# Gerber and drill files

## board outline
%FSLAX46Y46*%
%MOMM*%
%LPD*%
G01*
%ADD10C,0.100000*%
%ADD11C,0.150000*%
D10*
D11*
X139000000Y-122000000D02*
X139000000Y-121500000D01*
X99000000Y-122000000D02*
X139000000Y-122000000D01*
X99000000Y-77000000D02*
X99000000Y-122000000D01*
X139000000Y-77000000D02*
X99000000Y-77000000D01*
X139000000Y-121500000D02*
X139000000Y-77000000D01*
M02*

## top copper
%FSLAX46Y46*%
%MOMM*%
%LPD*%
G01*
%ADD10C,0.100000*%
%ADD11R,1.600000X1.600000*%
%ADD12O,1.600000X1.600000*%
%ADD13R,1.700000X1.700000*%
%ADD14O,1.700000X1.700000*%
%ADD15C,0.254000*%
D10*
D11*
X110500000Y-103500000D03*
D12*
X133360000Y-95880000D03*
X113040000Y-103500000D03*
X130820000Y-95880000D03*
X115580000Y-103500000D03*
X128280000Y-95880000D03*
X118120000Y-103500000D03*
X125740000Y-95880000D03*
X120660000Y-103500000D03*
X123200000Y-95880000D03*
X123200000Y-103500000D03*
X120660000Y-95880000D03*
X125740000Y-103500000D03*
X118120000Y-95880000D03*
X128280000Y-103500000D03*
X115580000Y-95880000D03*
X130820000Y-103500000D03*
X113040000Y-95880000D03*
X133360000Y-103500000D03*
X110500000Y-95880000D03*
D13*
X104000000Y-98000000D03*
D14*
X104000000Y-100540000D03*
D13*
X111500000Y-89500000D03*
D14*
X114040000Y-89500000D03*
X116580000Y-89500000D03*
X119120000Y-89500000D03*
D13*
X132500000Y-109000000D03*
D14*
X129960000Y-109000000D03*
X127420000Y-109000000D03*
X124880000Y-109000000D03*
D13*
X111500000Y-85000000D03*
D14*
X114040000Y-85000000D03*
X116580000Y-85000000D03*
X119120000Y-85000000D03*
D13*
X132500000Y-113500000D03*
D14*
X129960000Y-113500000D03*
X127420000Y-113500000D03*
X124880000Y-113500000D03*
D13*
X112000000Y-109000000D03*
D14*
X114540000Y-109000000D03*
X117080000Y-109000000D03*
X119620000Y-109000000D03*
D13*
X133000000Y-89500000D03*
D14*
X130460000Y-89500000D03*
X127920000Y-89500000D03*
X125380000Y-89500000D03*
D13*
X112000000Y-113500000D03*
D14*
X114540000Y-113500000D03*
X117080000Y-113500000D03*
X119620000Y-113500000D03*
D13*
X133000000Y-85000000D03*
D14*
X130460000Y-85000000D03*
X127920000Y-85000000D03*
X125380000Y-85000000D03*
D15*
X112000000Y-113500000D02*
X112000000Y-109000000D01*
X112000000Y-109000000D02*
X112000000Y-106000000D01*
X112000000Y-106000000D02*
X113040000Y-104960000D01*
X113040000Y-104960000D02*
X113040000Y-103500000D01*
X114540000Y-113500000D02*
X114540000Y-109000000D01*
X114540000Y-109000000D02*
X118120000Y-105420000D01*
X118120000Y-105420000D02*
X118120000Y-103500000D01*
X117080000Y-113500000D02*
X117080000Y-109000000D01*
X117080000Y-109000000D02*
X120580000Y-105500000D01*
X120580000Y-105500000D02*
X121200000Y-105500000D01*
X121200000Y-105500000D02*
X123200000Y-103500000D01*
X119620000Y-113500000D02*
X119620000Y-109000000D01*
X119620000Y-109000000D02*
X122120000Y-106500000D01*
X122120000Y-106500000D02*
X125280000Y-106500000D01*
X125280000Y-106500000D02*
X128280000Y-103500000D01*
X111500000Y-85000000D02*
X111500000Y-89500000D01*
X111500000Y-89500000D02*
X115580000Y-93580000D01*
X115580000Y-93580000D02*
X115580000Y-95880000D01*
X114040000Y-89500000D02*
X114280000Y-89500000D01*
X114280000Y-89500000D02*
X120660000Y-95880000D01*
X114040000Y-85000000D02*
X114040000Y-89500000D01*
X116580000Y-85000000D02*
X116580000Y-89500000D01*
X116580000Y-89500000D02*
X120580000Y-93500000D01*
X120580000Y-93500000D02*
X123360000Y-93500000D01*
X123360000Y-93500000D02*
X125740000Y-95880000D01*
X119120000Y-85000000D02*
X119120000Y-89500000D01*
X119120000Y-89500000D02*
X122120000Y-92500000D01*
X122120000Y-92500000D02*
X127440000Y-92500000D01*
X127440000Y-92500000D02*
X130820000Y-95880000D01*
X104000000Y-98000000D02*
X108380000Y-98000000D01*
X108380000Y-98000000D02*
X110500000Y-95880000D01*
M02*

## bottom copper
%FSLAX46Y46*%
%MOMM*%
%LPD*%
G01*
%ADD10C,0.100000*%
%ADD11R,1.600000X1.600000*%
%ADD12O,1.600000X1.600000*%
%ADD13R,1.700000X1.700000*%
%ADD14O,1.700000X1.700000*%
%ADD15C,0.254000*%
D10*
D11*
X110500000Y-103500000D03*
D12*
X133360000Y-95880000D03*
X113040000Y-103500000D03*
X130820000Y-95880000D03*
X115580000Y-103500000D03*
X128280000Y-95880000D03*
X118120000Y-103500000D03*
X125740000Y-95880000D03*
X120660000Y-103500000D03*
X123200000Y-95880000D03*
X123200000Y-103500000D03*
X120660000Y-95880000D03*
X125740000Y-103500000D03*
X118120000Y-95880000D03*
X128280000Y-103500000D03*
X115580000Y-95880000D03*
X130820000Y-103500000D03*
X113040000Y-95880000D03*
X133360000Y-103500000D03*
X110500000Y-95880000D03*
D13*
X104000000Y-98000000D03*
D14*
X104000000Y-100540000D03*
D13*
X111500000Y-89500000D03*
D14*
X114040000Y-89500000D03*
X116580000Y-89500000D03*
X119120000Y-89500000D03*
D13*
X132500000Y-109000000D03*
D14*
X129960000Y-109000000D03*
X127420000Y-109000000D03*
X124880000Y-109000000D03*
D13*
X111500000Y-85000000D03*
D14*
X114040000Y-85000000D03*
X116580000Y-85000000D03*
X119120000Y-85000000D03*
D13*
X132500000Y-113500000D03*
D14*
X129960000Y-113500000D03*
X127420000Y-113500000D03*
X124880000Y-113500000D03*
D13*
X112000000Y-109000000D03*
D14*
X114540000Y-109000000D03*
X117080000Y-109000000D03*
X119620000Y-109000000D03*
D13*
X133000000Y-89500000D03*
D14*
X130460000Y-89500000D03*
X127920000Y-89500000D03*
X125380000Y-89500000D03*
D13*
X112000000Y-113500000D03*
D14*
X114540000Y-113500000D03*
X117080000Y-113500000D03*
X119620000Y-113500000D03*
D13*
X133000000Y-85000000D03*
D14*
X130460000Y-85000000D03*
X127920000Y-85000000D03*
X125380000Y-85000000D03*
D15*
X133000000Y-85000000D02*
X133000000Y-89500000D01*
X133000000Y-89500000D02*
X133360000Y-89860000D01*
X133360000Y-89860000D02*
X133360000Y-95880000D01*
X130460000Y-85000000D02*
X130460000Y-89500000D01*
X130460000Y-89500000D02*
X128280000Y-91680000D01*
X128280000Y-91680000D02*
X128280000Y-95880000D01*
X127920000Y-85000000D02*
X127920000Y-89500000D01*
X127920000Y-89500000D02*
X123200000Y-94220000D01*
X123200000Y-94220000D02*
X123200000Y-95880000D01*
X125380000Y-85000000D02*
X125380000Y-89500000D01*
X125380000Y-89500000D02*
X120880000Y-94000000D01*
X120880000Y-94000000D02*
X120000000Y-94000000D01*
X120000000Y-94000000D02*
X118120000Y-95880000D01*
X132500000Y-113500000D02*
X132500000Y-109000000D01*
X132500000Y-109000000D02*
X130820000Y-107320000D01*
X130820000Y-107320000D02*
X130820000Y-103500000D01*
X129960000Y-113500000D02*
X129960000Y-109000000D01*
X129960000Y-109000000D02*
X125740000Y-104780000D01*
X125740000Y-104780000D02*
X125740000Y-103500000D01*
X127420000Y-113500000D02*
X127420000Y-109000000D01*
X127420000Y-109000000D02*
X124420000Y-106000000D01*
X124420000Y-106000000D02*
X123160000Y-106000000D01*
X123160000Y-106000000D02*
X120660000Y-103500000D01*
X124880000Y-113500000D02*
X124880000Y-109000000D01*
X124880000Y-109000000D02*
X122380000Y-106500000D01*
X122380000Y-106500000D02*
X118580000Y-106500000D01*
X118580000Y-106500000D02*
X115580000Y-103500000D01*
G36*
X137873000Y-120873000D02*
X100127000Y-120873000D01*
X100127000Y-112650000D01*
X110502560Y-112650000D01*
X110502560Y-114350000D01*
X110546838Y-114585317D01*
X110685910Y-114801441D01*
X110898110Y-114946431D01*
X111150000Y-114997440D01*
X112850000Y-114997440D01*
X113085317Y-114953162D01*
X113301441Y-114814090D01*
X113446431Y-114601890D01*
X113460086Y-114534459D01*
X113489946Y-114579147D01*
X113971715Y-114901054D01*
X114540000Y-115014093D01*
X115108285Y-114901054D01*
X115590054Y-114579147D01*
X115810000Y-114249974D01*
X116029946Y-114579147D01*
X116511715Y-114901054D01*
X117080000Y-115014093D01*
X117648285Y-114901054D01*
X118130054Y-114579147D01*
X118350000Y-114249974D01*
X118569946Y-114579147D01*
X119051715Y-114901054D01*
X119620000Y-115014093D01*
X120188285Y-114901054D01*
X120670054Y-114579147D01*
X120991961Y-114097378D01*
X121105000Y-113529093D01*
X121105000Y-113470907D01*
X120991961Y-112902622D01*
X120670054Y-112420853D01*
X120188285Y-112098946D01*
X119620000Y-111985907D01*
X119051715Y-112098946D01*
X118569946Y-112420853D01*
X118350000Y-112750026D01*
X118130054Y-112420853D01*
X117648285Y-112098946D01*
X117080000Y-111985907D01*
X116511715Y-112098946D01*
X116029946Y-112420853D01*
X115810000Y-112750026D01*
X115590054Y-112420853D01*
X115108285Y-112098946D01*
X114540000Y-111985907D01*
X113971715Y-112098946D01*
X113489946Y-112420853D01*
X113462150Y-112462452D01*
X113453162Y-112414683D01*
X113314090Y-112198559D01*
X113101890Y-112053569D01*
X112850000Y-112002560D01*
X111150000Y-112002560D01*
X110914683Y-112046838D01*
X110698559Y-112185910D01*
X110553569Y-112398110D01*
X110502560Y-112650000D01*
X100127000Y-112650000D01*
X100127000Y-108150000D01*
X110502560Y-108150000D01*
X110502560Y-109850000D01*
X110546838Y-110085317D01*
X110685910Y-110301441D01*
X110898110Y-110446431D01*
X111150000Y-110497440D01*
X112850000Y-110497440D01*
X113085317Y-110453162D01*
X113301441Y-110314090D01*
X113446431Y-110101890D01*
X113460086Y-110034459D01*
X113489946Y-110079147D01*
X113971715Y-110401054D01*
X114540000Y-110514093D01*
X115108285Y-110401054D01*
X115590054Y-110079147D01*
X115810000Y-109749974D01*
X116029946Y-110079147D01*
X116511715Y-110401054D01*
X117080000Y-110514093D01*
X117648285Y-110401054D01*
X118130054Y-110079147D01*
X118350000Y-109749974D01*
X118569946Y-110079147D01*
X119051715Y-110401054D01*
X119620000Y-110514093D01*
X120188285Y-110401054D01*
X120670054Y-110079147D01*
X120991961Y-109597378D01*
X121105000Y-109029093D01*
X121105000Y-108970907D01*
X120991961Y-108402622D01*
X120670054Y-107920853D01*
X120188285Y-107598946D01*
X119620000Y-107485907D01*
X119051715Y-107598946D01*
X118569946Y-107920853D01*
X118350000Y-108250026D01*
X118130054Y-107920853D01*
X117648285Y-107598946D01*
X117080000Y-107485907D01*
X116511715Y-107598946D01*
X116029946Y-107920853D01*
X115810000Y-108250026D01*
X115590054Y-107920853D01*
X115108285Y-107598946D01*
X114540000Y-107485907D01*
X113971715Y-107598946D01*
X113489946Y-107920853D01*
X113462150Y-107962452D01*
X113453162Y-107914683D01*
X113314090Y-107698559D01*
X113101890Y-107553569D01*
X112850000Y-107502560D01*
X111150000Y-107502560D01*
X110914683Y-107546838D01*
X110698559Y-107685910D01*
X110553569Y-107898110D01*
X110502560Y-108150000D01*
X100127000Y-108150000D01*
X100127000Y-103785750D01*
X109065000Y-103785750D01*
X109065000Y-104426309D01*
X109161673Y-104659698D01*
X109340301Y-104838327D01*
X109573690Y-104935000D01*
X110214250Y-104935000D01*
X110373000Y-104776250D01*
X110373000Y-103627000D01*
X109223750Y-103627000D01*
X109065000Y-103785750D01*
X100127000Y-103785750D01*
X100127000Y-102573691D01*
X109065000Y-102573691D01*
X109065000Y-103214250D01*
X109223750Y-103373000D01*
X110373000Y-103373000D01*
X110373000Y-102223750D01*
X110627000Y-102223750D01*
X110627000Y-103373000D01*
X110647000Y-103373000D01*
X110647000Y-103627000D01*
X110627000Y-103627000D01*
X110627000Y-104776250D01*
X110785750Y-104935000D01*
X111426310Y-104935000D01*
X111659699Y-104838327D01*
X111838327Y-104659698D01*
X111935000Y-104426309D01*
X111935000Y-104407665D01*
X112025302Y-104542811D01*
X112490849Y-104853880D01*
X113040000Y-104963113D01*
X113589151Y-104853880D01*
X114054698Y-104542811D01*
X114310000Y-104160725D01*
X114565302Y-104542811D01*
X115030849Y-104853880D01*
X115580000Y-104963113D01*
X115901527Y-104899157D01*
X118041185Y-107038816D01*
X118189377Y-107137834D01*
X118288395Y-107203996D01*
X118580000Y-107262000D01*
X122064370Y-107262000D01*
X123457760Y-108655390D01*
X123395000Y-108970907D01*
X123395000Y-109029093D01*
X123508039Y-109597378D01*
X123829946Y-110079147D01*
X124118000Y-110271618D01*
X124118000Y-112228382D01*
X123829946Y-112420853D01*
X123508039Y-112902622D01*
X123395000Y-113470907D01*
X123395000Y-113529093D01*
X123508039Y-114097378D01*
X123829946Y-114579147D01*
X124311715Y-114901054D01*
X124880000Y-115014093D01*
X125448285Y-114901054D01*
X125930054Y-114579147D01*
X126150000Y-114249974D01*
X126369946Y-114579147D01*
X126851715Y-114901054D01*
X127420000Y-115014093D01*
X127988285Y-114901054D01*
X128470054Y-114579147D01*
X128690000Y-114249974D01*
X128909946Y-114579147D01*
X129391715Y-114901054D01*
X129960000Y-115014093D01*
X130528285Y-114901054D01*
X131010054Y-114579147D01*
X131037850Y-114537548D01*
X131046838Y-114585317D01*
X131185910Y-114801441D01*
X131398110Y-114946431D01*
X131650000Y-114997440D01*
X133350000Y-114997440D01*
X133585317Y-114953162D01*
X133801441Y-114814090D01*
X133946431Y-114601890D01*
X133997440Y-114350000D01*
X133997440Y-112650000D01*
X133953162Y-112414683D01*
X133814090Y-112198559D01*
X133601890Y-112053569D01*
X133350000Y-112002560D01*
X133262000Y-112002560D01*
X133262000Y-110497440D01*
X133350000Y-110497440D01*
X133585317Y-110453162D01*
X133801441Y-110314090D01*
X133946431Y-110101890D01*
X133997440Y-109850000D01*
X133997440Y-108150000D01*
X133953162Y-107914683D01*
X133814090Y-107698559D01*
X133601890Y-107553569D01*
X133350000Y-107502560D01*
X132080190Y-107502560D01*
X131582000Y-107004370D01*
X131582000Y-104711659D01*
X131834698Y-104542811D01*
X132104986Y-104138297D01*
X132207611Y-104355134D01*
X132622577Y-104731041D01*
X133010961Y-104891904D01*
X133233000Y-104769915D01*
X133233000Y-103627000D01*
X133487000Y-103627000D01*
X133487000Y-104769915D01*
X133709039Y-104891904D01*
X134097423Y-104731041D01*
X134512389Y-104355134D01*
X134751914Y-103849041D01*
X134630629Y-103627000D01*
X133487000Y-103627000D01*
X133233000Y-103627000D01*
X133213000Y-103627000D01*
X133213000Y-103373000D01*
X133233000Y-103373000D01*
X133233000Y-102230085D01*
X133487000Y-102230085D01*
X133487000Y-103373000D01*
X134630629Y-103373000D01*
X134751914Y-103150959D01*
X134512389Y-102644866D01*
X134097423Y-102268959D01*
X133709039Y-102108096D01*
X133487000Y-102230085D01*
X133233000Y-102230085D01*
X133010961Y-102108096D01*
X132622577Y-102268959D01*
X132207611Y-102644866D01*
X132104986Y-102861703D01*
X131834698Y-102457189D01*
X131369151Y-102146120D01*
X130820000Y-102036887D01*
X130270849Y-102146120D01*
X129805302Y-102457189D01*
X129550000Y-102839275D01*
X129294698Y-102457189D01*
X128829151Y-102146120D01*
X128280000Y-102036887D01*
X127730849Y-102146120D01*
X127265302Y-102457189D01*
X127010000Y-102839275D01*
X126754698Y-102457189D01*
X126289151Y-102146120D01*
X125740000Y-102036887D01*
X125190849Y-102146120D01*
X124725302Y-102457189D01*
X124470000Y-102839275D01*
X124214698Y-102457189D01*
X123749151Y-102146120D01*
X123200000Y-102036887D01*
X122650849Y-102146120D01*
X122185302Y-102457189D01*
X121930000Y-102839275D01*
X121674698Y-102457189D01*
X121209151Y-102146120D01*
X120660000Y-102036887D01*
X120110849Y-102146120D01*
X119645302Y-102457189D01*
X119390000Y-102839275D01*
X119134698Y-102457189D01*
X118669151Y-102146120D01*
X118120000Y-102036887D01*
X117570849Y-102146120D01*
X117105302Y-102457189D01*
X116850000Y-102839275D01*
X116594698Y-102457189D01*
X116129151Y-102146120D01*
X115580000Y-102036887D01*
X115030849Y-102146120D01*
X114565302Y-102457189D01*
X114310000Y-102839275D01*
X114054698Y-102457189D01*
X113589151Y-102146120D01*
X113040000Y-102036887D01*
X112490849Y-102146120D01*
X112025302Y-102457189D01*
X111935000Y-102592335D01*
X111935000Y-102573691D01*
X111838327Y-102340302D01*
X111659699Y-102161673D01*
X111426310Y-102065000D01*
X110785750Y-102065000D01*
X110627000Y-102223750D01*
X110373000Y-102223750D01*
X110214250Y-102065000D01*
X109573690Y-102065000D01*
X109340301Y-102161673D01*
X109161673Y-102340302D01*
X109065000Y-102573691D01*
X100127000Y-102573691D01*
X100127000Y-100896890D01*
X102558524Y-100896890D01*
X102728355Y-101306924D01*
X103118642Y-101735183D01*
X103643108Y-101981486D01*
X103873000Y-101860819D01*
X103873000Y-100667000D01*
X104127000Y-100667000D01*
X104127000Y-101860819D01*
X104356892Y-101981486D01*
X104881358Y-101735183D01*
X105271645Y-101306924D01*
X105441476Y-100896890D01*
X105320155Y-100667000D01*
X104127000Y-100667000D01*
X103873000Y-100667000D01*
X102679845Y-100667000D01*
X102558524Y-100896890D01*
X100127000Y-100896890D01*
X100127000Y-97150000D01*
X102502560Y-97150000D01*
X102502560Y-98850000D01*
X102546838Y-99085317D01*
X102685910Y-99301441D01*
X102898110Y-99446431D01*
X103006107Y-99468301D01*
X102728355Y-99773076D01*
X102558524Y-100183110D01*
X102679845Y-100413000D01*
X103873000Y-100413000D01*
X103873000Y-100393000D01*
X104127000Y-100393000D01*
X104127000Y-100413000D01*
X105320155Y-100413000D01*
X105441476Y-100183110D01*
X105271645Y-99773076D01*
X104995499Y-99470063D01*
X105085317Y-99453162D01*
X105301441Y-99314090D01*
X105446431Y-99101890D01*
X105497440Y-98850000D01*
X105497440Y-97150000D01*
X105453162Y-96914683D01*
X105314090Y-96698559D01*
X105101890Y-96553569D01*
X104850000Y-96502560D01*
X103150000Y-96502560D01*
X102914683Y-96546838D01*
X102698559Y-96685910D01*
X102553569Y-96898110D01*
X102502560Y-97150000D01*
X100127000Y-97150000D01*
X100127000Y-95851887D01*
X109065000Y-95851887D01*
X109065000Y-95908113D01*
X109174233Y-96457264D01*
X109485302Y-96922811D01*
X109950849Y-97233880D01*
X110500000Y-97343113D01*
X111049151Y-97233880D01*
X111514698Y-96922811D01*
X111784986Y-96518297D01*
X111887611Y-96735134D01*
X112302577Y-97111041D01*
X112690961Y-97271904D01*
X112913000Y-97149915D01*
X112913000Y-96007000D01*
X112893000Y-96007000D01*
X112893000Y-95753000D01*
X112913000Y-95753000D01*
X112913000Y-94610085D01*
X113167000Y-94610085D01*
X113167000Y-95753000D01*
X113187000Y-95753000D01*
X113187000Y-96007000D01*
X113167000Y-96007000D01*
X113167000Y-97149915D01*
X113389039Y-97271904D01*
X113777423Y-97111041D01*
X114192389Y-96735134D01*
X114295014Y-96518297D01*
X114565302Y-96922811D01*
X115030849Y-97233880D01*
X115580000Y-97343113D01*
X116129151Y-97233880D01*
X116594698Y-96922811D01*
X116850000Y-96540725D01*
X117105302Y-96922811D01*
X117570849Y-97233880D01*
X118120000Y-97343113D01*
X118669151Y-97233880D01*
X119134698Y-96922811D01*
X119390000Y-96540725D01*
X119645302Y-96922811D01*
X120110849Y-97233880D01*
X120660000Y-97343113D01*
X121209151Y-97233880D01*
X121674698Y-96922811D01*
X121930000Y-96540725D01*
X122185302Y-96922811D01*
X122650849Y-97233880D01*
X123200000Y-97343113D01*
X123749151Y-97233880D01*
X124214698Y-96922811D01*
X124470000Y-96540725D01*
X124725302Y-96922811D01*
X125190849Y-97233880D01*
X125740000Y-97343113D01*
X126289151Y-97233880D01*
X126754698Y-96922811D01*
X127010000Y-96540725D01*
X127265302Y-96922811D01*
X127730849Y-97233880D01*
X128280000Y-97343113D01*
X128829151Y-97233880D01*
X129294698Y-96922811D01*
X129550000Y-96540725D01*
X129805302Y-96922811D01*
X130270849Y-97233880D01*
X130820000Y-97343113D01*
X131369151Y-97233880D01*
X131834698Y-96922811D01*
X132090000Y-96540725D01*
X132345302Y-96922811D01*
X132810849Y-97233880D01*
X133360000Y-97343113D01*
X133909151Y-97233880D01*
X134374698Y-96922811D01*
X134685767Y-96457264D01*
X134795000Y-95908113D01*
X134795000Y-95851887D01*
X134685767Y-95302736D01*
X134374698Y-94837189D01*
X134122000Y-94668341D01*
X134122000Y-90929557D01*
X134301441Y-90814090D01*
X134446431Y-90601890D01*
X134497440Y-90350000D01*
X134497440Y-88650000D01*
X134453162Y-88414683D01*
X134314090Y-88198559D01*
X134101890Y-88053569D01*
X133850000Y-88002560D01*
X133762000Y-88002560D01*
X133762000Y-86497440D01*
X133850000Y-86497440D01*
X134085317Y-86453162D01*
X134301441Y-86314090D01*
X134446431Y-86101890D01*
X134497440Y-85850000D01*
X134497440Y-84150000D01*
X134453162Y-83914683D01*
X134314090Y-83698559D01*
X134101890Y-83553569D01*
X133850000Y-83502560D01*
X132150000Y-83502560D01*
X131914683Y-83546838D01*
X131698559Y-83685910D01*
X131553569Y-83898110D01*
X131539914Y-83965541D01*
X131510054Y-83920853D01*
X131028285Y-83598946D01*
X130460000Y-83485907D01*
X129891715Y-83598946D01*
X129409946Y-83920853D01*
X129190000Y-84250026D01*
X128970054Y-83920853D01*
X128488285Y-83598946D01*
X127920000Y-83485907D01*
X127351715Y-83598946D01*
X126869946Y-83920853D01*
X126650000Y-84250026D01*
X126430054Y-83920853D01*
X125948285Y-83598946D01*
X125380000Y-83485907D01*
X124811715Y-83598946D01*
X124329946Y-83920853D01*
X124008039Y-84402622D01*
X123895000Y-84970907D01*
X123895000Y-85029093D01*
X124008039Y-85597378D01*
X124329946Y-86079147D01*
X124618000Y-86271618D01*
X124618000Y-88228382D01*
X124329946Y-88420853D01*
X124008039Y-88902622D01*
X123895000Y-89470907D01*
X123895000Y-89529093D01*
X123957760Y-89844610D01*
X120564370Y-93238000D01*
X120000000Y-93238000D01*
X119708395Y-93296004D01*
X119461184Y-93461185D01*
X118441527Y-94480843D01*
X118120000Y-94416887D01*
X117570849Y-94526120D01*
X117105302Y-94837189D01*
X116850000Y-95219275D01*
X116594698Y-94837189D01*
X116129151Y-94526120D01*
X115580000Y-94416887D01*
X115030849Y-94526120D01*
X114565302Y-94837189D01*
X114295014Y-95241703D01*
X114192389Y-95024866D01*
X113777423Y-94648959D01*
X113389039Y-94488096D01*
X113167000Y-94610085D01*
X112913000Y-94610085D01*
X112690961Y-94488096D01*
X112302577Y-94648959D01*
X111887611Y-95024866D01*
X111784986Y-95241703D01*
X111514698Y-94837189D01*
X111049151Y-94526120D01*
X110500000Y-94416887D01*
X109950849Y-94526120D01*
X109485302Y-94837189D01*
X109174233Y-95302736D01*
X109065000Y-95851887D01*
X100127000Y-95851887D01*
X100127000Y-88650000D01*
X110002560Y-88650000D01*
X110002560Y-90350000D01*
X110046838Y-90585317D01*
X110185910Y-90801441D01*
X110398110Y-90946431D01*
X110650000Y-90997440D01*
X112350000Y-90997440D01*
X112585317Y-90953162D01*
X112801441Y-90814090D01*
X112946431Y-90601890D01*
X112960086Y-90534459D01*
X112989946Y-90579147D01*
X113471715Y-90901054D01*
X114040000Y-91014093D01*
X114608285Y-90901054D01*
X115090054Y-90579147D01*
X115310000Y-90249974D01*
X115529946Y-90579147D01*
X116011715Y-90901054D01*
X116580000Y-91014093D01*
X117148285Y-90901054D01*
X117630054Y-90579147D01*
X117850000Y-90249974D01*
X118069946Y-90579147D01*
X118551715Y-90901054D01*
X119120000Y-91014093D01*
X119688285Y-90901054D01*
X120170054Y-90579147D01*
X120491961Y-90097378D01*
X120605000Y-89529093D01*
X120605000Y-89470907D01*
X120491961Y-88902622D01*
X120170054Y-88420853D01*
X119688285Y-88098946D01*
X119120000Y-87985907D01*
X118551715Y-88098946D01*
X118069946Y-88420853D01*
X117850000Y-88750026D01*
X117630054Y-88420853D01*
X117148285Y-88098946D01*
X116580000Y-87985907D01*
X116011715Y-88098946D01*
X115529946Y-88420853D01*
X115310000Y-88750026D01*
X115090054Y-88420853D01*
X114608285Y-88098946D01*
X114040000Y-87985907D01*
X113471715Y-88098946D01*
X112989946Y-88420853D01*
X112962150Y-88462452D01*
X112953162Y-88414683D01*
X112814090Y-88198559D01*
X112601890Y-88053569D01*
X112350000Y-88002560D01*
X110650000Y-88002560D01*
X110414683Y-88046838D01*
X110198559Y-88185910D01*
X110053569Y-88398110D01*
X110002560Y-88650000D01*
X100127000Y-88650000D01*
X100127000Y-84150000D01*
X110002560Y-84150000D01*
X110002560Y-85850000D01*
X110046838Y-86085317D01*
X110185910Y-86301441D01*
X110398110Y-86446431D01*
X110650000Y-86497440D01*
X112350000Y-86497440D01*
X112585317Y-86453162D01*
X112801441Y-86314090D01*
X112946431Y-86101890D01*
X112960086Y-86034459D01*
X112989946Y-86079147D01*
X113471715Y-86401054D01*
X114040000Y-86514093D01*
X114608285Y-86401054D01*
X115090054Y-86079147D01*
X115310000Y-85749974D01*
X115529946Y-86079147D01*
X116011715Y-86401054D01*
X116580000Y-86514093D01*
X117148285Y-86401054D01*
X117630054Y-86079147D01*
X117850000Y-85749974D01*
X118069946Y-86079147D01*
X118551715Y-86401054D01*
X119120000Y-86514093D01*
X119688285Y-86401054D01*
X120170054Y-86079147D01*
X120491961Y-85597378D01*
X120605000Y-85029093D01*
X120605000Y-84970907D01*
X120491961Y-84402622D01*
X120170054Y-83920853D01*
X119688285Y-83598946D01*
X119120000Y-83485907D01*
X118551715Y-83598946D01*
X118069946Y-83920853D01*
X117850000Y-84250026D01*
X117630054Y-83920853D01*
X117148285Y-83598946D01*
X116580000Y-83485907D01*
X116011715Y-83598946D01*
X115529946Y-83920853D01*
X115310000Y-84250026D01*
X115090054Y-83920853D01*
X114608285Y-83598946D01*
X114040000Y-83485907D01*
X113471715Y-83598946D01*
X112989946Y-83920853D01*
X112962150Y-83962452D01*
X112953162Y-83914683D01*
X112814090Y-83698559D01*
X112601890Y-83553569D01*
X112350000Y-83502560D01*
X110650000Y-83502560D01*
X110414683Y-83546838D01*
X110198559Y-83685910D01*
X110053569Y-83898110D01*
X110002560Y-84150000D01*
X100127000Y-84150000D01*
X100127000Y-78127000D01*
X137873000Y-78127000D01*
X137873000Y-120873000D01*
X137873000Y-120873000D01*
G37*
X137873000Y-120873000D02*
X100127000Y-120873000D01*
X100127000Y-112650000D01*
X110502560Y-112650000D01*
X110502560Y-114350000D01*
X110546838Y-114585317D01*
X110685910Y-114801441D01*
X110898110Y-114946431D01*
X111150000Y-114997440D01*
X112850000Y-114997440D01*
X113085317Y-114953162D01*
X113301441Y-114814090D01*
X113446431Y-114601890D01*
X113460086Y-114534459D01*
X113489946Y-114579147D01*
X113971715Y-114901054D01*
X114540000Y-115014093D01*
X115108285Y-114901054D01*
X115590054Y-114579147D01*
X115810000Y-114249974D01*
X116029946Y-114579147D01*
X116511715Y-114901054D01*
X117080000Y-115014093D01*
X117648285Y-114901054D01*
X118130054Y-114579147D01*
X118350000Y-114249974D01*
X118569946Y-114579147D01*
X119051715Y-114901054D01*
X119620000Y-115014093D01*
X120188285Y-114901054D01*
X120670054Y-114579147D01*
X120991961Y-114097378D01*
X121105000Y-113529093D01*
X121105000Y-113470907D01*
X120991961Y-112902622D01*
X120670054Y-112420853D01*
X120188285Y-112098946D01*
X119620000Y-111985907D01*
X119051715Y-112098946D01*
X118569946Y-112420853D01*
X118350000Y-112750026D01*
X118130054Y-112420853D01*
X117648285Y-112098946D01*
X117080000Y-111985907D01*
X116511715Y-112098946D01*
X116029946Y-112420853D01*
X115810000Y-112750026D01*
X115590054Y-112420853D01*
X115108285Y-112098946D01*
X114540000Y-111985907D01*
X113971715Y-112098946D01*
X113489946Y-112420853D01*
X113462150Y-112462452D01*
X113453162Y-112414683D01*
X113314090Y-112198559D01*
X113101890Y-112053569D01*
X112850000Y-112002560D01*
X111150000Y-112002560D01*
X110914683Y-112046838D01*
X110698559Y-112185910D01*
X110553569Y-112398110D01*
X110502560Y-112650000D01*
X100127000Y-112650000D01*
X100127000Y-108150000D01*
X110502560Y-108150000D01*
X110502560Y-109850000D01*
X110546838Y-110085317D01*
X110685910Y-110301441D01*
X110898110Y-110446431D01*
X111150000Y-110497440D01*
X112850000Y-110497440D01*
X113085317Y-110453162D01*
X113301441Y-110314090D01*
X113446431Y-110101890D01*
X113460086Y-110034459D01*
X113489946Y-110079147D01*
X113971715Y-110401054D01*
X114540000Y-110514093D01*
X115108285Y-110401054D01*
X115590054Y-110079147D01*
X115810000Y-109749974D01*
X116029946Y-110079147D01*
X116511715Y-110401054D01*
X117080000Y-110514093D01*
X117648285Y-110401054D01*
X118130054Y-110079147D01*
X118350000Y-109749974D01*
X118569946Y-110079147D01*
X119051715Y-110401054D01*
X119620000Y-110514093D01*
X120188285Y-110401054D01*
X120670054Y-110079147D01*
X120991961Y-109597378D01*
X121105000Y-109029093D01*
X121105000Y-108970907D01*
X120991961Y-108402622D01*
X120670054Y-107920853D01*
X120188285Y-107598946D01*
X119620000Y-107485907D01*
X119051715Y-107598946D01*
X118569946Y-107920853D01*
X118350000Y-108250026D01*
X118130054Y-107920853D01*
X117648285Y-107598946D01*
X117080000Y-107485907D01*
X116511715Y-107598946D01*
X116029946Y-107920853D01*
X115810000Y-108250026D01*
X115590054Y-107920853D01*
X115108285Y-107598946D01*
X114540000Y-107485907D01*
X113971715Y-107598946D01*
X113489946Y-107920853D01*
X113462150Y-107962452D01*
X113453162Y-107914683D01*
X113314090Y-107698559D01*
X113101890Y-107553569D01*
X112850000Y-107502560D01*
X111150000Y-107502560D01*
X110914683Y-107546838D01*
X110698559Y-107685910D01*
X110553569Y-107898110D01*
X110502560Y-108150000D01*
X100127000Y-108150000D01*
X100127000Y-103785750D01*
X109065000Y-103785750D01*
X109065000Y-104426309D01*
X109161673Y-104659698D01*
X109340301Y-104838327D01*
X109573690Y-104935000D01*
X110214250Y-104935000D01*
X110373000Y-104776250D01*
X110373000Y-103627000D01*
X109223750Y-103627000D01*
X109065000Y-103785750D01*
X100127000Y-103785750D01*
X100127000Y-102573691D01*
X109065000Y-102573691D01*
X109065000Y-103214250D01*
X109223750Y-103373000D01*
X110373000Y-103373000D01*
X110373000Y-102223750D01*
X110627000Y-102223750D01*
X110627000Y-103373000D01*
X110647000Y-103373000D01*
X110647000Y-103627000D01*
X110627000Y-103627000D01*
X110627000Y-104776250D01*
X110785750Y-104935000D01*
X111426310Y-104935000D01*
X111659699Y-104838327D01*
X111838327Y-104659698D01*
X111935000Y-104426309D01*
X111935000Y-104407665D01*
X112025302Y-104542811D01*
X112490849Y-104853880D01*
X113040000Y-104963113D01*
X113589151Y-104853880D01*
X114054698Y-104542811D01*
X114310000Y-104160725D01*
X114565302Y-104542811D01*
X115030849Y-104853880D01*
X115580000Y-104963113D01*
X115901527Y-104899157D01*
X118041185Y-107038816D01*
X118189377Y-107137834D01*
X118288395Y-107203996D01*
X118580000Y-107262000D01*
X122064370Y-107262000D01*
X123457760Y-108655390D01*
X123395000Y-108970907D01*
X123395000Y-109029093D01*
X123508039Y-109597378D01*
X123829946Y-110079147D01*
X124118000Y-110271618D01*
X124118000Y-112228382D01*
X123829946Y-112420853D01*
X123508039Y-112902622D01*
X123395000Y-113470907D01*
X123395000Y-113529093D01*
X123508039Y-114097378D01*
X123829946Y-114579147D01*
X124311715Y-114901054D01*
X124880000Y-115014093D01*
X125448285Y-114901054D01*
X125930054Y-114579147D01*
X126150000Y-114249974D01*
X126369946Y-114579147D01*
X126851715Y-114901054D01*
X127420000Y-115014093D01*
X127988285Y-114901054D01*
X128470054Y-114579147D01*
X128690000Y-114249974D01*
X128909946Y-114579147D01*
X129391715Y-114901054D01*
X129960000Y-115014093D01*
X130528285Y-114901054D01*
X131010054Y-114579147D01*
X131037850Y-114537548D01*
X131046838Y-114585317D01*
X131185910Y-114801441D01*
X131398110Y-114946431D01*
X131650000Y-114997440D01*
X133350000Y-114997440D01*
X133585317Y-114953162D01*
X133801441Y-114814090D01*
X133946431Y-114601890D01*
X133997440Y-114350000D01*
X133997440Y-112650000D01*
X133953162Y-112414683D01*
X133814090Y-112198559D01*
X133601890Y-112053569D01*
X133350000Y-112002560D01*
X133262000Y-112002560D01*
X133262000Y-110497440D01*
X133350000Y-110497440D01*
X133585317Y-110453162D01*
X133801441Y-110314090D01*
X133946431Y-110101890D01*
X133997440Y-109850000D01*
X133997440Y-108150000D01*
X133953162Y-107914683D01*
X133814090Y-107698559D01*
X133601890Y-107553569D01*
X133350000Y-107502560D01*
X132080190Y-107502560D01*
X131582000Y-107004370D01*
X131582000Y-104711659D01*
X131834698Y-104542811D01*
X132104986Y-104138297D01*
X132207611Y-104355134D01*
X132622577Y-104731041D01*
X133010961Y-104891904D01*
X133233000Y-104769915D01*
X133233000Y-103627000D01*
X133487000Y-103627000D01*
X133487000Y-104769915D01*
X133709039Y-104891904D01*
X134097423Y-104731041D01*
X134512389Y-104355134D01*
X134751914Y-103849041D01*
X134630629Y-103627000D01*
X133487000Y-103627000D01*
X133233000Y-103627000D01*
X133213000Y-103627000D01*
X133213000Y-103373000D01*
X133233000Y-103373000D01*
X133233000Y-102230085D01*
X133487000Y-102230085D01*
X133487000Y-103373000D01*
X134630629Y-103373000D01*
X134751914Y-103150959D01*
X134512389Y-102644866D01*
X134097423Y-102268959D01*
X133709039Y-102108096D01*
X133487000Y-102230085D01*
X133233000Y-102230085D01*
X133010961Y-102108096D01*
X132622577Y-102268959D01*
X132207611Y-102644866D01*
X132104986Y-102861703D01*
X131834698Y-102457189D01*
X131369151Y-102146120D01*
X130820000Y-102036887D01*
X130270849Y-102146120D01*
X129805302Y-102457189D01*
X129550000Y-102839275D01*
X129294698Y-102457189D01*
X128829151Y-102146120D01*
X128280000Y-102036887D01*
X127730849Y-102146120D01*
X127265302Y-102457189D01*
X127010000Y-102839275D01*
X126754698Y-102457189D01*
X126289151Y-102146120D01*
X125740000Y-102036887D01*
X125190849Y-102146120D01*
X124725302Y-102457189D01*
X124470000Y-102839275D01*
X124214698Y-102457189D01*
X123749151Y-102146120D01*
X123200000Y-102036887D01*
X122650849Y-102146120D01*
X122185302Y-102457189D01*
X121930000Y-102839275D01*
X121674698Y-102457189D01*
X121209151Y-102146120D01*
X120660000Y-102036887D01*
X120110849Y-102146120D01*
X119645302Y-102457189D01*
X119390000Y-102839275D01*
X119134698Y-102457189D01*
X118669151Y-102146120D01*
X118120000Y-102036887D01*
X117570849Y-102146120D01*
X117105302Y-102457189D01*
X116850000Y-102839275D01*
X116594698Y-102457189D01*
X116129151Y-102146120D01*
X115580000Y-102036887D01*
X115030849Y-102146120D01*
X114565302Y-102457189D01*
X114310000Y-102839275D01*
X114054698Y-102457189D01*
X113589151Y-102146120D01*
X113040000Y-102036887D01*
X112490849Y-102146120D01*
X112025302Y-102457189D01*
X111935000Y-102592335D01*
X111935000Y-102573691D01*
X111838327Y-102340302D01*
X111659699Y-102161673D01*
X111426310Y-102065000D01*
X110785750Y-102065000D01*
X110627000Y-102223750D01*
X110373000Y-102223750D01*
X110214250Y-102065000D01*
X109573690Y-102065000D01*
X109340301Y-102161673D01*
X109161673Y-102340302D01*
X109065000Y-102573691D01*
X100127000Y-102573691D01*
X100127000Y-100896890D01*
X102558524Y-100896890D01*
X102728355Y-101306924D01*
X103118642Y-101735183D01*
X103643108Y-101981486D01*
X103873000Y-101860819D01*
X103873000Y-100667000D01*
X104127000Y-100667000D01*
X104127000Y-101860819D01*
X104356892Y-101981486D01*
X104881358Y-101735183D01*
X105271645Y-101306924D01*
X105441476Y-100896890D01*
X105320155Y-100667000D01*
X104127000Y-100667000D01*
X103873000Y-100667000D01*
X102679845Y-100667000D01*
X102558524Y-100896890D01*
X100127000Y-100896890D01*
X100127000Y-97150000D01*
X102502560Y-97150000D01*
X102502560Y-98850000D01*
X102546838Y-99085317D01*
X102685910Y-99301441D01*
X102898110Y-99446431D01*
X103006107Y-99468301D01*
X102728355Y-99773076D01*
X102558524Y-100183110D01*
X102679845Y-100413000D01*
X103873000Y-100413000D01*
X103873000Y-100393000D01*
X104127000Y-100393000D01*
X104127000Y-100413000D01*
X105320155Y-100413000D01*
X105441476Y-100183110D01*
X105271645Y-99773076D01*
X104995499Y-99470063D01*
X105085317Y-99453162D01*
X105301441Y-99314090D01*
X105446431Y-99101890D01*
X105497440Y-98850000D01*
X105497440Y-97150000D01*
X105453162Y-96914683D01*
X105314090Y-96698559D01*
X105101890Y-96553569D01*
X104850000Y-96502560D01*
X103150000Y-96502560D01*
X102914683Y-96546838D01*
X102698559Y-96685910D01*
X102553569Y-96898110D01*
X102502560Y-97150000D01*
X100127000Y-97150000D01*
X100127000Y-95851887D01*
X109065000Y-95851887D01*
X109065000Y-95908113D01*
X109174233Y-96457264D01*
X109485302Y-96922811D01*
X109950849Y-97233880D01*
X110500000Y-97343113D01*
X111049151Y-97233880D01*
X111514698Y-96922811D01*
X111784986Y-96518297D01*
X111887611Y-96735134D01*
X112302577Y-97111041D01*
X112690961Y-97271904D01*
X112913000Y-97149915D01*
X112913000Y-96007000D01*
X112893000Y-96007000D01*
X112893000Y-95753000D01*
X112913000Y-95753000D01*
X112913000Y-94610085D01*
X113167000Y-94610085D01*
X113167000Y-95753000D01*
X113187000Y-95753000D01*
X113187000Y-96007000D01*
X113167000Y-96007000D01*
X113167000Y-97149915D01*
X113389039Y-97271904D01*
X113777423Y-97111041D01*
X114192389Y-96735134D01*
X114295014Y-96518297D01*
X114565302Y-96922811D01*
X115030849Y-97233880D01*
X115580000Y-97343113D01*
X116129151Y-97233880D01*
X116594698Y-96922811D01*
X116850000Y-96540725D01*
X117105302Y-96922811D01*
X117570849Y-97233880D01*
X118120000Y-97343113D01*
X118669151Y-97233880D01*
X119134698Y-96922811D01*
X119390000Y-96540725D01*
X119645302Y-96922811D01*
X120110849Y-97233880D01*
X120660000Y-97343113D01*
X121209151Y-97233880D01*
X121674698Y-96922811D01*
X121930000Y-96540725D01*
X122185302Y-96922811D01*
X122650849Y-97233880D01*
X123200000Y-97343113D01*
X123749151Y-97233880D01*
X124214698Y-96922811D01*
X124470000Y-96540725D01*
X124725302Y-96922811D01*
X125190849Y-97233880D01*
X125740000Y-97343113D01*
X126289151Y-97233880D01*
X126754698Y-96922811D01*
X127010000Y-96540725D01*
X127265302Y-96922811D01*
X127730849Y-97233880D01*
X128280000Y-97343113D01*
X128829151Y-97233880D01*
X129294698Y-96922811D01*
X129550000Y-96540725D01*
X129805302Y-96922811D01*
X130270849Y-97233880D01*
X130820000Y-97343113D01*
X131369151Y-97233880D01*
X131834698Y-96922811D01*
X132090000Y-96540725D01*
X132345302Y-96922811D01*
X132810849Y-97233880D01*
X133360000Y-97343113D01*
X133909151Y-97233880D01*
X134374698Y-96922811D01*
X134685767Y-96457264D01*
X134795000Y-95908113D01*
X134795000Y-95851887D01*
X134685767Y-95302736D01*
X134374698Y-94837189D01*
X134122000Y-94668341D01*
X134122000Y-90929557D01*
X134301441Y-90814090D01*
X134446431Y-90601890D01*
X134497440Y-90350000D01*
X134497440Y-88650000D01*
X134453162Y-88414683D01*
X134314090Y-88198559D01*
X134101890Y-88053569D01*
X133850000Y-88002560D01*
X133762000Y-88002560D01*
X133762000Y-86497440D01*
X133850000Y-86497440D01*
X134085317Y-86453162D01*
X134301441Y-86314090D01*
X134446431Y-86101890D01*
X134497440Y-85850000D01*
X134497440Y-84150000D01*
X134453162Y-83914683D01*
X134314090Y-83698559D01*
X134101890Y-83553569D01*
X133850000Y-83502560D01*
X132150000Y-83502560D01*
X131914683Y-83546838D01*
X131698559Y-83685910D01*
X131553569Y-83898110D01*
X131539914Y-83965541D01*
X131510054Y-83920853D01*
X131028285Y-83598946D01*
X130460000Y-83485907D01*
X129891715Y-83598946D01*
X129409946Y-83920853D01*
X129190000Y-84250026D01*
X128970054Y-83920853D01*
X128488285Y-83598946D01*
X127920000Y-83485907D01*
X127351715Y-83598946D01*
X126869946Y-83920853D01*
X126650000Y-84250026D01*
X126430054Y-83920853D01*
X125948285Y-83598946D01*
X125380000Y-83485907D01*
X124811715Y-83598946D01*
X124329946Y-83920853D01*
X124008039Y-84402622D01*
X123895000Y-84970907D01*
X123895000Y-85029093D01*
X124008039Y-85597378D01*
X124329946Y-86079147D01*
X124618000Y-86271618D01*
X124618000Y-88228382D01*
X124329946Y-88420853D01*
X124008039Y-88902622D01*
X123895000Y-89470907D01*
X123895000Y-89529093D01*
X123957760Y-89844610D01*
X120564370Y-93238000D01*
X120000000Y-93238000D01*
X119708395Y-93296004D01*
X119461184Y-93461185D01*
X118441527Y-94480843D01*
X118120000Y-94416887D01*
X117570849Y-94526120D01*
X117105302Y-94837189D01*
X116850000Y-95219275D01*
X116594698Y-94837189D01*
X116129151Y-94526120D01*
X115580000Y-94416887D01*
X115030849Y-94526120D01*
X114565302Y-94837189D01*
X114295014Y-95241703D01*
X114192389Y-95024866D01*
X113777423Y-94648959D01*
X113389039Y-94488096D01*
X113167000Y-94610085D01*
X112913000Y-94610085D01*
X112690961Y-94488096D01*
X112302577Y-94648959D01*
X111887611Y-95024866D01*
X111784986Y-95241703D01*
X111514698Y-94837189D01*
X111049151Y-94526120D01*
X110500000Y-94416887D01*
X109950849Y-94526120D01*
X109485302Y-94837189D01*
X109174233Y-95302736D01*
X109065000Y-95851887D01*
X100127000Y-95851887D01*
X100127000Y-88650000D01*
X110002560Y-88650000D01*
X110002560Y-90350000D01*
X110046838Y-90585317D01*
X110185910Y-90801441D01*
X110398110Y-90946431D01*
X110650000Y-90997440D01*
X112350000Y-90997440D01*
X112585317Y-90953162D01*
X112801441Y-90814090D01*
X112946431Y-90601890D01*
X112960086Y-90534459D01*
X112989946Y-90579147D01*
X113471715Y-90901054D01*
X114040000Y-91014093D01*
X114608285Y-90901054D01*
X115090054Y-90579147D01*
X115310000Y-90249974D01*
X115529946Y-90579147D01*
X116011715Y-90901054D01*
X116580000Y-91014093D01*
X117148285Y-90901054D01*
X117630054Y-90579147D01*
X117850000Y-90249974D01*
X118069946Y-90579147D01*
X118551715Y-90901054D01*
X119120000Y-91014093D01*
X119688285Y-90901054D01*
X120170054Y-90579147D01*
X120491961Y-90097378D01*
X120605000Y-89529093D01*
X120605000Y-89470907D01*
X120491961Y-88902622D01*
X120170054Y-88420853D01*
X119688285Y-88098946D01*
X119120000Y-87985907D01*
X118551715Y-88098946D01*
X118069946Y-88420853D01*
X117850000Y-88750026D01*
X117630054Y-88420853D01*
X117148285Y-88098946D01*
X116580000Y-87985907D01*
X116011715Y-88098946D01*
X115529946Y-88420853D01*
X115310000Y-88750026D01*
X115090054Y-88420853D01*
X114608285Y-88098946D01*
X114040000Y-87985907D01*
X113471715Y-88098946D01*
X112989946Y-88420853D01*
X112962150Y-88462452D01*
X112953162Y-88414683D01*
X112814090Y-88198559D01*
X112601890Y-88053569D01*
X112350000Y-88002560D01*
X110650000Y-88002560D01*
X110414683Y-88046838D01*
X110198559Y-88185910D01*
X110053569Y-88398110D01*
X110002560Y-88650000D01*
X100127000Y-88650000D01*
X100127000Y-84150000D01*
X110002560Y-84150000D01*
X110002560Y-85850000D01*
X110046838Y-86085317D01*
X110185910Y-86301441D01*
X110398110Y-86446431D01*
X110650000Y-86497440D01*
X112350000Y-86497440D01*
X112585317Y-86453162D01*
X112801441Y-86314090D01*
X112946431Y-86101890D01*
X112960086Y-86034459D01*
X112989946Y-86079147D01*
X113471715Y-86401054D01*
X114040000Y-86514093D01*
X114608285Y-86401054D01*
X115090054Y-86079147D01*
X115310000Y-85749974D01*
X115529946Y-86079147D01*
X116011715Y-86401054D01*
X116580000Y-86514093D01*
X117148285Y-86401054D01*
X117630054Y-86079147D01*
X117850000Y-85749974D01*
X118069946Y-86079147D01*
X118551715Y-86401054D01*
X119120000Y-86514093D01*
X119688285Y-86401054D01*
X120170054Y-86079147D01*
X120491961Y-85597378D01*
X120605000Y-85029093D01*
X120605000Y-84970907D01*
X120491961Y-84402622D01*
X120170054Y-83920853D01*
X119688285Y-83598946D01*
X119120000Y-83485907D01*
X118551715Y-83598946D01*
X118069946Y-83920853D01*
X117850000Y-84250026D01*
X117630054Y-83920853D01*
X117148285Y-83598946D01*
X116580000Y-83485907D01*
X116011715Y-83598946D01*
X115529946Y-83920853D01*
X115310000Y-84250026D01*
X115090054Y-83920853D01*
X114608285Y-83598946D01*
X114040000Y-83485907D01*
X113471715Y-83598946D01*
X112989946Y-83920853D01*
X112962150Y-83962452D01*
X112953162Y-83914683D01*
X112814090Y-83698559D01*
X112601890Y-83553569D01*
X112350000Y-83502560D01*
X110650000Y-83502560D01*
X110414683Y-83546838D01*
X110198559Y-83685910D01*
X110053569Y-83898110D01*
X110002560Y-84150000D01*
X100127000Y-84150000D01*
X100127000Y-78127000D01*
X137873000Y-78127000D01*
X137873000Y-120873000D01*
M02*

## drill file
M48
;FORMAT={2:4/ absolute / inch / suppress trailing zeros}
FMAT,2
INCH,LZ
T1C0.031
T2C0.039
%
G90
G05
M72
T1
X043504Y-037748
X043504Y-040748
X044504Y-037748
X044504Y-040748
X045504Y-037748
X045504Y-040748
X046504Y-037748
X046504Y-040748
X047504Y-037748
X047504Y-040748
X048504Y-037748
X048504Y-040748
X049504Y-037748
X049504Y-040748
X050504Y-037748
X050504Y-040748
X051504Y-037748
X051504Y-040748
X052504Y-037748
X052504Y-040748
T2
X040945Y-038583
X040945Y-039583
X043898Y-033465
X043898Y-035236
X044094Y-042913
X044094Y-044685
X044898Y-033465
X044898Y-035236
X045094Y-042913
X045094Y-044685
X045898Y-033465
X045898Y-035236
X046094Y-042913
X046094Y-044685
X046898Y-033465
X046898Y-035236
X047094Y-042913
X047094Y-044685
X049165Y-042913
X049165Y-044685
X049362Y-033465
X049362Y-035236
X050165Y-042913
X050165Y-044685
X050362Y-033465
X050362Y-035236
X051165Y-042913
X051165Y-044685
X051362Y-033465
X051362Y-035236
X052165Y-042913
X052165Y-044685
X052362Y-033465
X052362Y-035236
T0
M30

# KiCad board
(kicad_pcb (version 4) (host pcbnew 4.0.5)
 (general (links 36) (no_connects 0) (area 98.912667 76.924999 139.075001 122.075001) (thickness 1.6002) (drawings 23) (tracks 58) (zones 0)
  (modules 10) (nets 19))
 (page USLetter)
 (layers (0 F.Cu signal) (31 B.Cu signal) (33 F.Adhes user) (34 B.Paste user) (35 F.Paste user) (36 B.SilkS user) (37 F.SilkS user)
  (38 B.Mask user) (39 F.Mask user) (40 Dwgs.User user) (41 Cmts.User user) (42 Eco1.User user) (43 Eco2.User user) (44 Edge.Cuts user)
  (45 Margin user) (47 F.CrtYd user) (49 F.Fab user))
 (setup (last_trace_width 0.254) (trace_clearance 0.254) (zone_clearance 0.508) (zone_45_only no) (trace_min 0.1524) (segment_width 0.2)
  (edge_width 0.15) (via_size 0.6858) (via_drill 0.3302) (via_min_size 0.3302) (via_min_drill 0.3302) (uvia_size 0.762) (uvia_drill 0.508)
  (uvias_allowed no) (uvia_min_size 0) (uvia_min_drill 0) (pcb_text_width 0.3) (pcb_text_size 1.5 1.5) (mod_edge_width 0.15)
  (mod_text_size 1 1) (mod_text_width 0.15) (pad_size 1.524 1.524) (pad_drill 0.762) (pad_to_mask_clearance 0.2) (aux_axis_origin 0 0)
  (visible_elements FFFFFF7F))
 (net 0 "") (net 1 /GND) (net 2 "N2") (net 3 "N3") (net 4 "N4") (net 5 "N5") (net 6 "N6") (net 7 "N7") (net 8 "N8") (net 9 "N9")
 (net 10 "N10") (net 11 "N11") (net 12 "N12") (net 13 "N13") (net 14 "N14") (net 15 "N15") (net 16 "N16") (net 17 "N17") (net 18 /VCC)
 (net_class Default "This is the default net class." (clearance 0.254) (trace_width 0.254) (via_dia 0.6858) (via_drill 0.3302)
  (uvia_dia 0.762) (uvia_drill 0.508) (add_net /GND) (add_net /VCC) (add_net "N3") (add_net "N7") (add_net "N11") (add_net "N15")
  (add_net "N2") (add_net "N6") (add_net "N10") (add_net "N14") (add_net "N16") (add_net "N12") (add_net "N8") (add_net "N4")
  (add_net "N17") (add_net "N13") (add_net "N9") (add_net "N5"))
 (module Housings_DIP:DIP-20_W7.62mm (layer F.Cu) (at 110.5 103.5 90)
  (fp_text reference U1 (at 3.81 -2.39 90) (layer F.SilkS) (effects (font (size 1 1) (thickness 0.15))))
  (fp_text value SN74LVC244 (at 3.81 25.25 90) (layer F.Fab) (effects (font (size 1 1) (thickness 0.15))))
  (pad 1 thru_hole rect (at 0 0 90) (size 1.6 1.6) (drill 0.8) (layers *.Cu *.Mask) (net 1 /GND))
  (pad 11 thru_hole oval (at 7.62 22.86 90) (size 1.6 1.6) (drill 0.8) (layers *.Cu *.Mask) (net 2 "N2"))
  (pad 2 thru_hole oval (at 0 2.54 90) (size 1.6 1.6) (drill 0.8) (layers *.Cu *.Mask) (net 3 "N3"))
  (pad 12 thru_hole oval (at 7.62 20.32 90) (size 1.6 1.6) (drill 0.8) (layers *.Cu *.Mask) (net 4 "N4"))
  (pad 3 thru_hole oval (at 0 5.08 90) (size 1.6 1.6) (drill 0.8) (layers *.Cu *.Mask) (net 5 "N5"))
  (pad 13 thru_hole oval (at 7.62 17.78 90) (size 1.6 1.6) (drill 0.8) (layers *.Cu *.Mask) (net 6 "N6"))
  (pad 4 thru_hole oval (at 0 7.62 90) (size 1.6 1.6) (drill 0.8) (layers *.Cu *.Mask) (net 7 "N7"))
  (pad 14 thru_hole oval (at 7.62 15.24 90) (size 1.6 1.6) (drill 0.8) (layers *.Cu *.Mask) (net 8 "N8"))
  (pad 5 thru_hole oval (at 0 10.16 90) (size 1.6 1.6) (drill 0.8) (layers *.Cu *.Mask) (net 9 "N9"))
  (pad 15 thru_hole oval (at 7.62 12.7 90) (size 1.6 1.6) (drill 0.8) (layers *.Cu *.Mask) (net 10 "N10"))
  (pad 6 thru_hole oval (at 0 12.7 90) (size 1.6 1.6) (drill 0.8) (layers *.Cu *.Mask) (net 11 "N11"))
  (pad 16 thru_hole oval (at 7.62 10.16 90) (size 1.6 1.6) (drill 0.8) (layers *.Cu *.Mask) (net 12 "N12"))
  (pad 7 thru_hole oval (at 0 15.24 90) (size 1.6 1.6) (drill 0.8) (layers *.Cu *.Mask) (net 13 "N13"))
  (pad 17 thru_hole oval (at 7.62 7.62 90) (size 1.6 1.6) (drill 0.8) (layers *.Cu *.Mask) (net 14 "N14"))
  (pad 8 thru_hole oval (at 0 17.78 90) (size 1.6 1.6) (drill 0.8) (layers *.Cu *.Mask) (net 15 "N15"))
  (pad 18 thru_hole oval (at 7.62 5.08 90) (size 1.6 1.6) (drill 0.8) (layers *.Cu *.Mask) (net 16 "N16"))
  (pad 9 thru_hole oval (at 0 20.32 90) (size 1.6 1.6) (drill 0.8) (layers *.Cu *.Mask) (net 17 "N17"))
  (pad 19 thru_hole oval (at 7.62 2.54 90) (size 1.6 1.6) (drill 0.8) (layers *.Cu *.Mask) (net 1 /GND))
  (pad 10 thru_hole oval (at 0 22.86 90) (size 1.6 1.6) (drill 0.8) (layers *.Cu *.Mask) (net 1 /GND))
  (pad 20 thru_hole oval (at 7.62 0 90) (size 1.6 1.6) (drill 0.8) (layers *.Cu *.Mask) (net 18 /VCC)))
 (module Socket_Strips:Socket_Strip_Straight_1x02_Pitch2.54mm (layer F.Cu) (at 104 98)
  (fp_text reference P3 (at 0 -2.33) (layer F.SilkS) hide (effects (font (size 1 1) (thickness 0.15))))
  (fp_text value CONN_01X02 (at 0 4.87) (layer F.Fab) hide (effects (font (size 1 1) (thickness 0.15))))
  (pad 1 thru_hole rect (at 0 0) (size 1.7 1.7) (drill 1) (layers *.Cu *.Mask) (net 18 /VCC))
  (pad 2 thru_hole oval (at 0 2.54) (size 1.7 1.7) (drill 1) (layers *.Cu *.Mask) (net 1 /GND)))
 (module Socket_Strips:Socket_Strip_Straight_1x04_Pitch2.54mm (layer F.Cu) (at 111.5 89.5 90)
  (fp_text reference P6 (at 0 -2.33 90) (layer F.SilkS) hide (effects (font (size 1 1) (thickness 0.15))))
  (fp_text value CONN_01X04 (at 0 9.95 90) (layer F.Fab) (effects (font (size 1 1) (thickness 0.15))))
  (pad 1 thru_hole rect (at 0 0 90) (size 1.7 1.7) (drill 1) (layers *.Cu *.Mask) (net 16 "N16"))
  (pad 2 thru_hole oval (at 0 2.54 90) (size 1.7 1.7) (drill 1) (layers *.Cu *.Mask) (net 12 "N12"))
  (pad 3 thru_hole oval (at 0 5.08 90) (size 1.7 1.7) (drill 1) (layers *.Cu *.Mask) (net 8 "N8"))
  (pad 4 thru_hole oval (at 0 7.62 90) (size 1.7 1.7) (drill 1) (layers *.Cu *.Mask) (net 4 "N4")))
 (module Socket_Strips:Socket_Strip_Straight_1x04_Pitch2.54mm (layer F.Cu) (at 132.5 109 270)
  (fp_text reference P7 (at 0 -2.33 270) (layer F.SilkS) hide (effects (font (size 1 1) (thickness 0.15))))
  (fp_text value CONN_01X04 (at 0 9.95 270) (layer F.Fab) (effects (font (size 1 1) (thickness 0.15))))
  (pad 1 thru_hole rect (at 0 0 270) (size 1.7 1.7) (drill 1) (layers *.Cu *.Mask) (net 17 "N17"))
  (pad 2 thru_hole oval (at 0 2.54 270) (size 1.7 1.7) (drill 1) (layers *.Cu *.Mask) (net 13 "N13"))
  (pad 3 thru_hole oval (at 0 5.08 270) (size 1.7 1.7) (drill 1) (layers *.Cu *.Mask) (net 9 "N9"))
  (pad 4 thru_hole oval (at 0 7.62 270) (size 1.7 1.7) (drill 1) (layers *.Cu *.Mask) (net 5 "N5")))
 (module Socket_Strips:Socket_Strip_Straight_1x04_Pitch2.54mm (layer F.Cu) (at 111.5 85 90)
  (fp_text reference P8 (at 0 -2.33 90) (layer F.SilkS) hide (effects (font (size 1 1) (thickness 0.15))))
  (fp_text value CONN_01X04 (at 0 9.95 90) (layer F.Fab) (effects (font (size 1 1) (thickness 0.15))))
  (pad 1 thru_hole rect (at 0 0 90) (size 1.7 1.7) (drill 1) (layers *.Cu *.Mask) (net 16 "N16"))
  (pad 2 thru_hole oval (at 0 2.54 90) (size 1.7 1.7) (drill 1) (layers *.Cu *.Mask) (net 12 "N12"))
  (pad 3 thru_hole oval (at 0 5.08 90) (size 1.7 1.7) (drill 1) (layers *.Cu *.Mask) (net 8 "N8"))
  (pad 4 thru_hole oval (at 0 7.62 90) (size 1.7 1.7) (drill 1) (layers *.Cu *.Mask) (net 4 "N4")))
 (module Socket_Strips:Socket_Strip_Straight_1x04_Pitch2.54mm (layer F.Cu) (at 132.5 113.5 270)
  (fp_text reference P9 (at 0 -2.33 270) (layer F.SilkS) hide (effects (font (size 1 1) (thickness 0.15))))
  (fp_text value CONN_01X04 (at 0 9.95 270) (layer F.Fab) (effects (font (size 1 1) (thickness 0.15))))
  (pad 1 thru_hole rect (at 0 0 270) (size 1.7 1.7) (drill 1) (layers *.Cu *.Mask) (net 17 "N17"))
  (pad 2 thru_hole oval (at 0 2.54 270) (size 1.7 1.7) (drill 1) (layers *.Cu *.Mask) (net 13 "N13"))
  (pad 3 thru_hole oval (at 0 5.08 270) (size 1.7 1.7) (drill 1) (layers *.Cu *.Mask) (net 9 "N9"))
  (pad 4 thru_hole oval (at 0 7.62 270) (size 1.7 1.7) (drill 1) (layers *.Cu *.Mask) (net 5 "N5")))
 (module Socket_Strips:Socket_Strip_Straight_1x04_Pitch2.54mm (layer F.Cu) (at 112 109 90)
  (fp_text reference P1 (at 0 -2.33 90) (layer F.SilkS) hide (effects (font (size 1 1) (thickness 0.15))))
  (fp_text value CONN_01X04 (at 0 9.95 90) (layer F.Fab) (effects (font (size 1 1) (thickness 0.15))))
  (pad 1 thru_hole rect (at 0 0 90) (size 1.7 1.7) (drill 1) (layers *.Cu *.Mask) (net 3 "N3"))
  (pad 2 thru_hole oval (at 0 2.54 90) (size 1.7 1.7) (drill 1) (layers *.Cu *.Mask) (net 7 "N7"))
  (pad 3 thru_hole oval (at 0 5.08 90) (size 1.7 1.7) (drill 1) (layers *.Cu *.Mask) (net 11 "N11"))
  (pad 4 thru_hole oval (at 0 7.62 90) (size 1.7 1.7) (drill 1) (layers *.Cu *.Mask) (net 15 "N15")))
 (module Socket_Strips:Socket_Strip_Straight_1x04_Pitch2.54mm (layer F.Cu) (at 133 89.5 270)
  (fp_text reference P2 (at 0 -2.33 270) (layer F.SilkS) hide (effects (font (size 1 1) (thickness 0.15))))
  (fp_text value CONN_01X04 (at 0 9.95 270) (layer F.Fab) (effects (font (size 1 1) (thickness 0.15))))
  (pad 1 thru_hole rect (at 0 0 270) (size 1.7 1.7) (drill 1) (layers *.Cu *.Mask) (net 2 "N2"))
  (pad 2 thru_hole oval (at 0 2.54 270) (size 1.7 1.7) (drill 1) (layers *.Cu *.Mask) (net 6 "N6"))
  (pad 3 thru_hole oval (at 0 5.08 270) (size 1.7 1.7) (drill 1) (layers *.Cu *.Mask) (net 10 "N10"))
  (pad 4 thru_hole oval (at 0 7.62 270) (size 1.7 1.7) (drill 1) (layers *.Cu *.Mask) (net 14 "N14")))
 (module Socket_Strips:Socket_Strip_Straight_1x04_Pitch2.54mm (layer F.Cu) (at 112 113.5 90)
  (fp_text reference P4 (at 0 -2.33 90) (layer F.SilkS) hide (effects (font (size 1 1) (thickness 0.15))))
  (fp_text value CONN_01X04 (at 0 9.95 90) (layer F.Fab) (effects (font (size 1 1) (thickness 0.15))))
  (pad 1 thru_hole rect (at 0 0 90) (size 1.7 1.7) (drill 1) (layers *.Cu *.Mask) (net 3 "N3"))
  (pad 2 thru_hole oval (at 0 2.54 90) (size 1.7 1.7) (drill 1) (layers *.Cu *.Mask) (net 7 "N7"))
  (pad 3 thru_hole oval (at 0 5.08 90) (size 1.7 1.7) (drill 1) (layers *.Cu *.Mask) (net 11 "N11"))
  (pad 4 thru_hole oval (at 0 7.62 90) (size 1.7 1.7) (drill 1) (layers *.Cu *.Mask) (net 15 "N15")))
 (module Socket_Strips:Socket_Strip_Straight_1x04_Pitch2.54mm (layer F.Cu) (at 133 85 270)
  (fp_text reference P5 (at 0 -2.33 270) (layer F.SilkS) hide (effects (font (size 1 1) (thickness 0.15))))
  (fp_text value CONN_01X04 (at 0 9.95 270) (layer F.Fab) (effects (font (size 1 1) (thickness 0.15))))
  (pad 1 thru_hole rect (at 0 0 270) (size 1.7 1.7) (drill 1) (layers *.Cu *.Mask) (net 2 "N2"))
  (pad 2 thru_hole oval (at 0 2.54 270) (size 1.7 1.7) (drill 1) (layers *.Cu *.Mask) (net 6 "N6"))
  (pad 3 thru_hole oval (at 0 5.08 270) (size 1.7 1.7) (drill 1) (layers *.Cu *.Mask) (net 10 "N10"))
  (pad 4 thru_hole oval (at 0 7.62 270) (size 1.7 1.7) (drill 1) (layers *.Cu *.Mask) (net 14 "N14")))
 (gr_line (start 139 122) (end 139 121.5) (angle 90) (layer Edge.Cuts) (width 0.15))
 (gr_line (start 99 122) (end 139 122) (angle 90) (layer Edge.Cuts) (width 0.15))
 (gr_line (start 99 77) (end 99 122) (angle 90) (layer Edge.Cuts) (width 0.15))
 (gr_line (start 139 77) (end 99 77) (angle 90) (layer Edge.Cuts) (width 0.15))
 (gr_line (start 139 121.5) (end 139 77) (angle 90) (layer Edge.Cuts) (width 0.15))
 (segment (start 112 113.5) (end 112 109) (width 0.254) (layer F.Cu) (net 3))
 (segment (start 112 109) (end 112 106) (width 0.254) (layer F.Cu) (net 3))
 (segment (start 112 106) (end 113.04 104.96) (width 0.254) (layer F.Cu) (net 3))
 (segment (start 113.04 104.96) (end 113.04 103.5) (width 0.254) (layer F.Cu) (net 3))
 (segment (start 114.54 113.5) (end 114.54 109) (width 0.254) (layer F.Cu) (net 7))
 (segment (start 114.54 109) (end 118.12 105.42) (width 0.254) (layer F.Cu) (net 7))
 (segment (start 118.12 105.42) (end 118.12 103.5) (width 0.254) (layer F.Cu) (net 7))
 (segment (start 117.08 113.5) (end 117.08 109) (width 0.254) (layer F.Cu) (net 11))
 (segment (start 117.08 109) (end 120.58 105.5) (width 0.254) (layer F.Cu) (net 11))
 (segment (start 120.58 105.5) (end 121.2 105.5) (width 0.254) (layer F.Cu) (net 11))
 (segment (start 121.2 105.5) (end 123.2 103.5) (width 0.254) (layer F.Cu) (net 11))
 (segment (start 119.62 113.5) (end 119.62 109) (width 0.254) (layer F.Cu) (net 15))
 (segment (start 119.62 109) (end 122.12 106.5) (width 0.254) (layer F.Cu) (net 15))
 (segment (start 122.12 106.5) (end 125.28 106.5) (width 0.254) (layer F.Cu) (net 15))
 (segment (start 125.28 106.5) (end 128.28 103.5) (width 0.254) (layer F.Cu) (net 15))
 (segment (start 133 85) (end 133 89.5) (width 0.254) (layer B.Cu) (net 2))
 (segment (start 133 89.5) (end 133.36 89.86) (width 0.254) (layer B.Cu) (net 2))
 (segment (start 133.36 89.86) (end 133.36 95.88) (width 0.254) (layer B.Cu) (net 2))
 (segment (start 130.46 85) (end 130.46 89.5) (width 0.254) (layer B.Cu) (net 6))
 (segment (start 130.46 89.5) (end 128.28 91.68) (width 0.254) (layer B.Cu) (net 6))
 (segment (start 128.28 91.68) (end 128.28 95.88) (width 0.254) (layer B.Cu) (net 6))
 (segment (start 127.92 85) (end 127.92 89.5) (width 0.254) (layer B.Cu) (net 10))
 (segment (start 127.92 89.5) (end 123.2 94.22) (width 0.254) (layer B.Cu) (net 10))
 (segment (start 123.2 94.22) (end 123.2 95.88) (width 0.254) (layer B.Cu) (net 10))
 (segment (start 125.38 85) (end 125.38 89.5) (width 0.254) (layer B.Cu) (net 14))
 (segment (start 125.38 89.5) (end 120.88 94) (width 0.254) (layer B.Cu) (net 14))
 (segment (start 120.88 94) (end 120 94) (width 0.254) (layer B.Cu) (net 14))
 (segment (start 120 94) (end 118.12 95.88) (width 0.254) (layer B.Cu) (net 14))
 (segment (start 111.5 85) (end 111.5 89.5) (width 0.254) (layer F.Cu) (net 16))
 (segment (start 111.5 89.5) (end 115.58 93.58) (width 0.254) (layer F.Cu) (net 16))
 (segment (start 115.58 93.58) (end 115.58 95.88) (width 0.254) (layer F.Cu) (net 16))
 (segment (start 114.04 89.5) (end 114.28 89.5) (width 0.254) (layer F.Cu) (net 12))
 (segment (start 114.28 89.5) (end 120.66 95.88) (width 0.254) (layer F.Cu) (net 12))
 (segment (start 114.04 85) (end 114.04 89.5) (width 0.254) (layer F.Cu) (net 12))
 (segment (start 116.58 85) (end 116.58 89.5) (width 0.254) (layer F.Cu) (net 8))
 (segment (start 116.58 89.5) (end 120.58 93.5) (width 0.254) (layer F.Cu) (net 8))
 (segment (start 120.58 93.5) (end 123.36 93.5) (width 0.254) (layer F.Cu) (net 8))
 (segment (start 123.36 93.5) (end 125.74 95.88) (width 0.254) (layer F.Cu) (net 8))
 (segment (start 119.12 85) (end 119.12 89.5) (width 0.254) (layer F.Cu) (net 4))
 (segment (start 119.12 89.5) (end 122.12 92.5) (width 0.254) (layer F.Cu) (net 4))
 (segment (start 122.12 92.5) (end 127.44 92.5) (width 0.254) (layer F.Cu) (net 4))
 (segment (start 127.44 92.5) (end 130.82 95.88) (width 0.254) (layer F.Cu) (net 4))
 (segment (start 132.5 113.5) (end 132.5 109) (width 0.254) (layer B.Cu) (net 17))
 (segment (start 132.5 109) (end 130.82 107.32) (width 0.254) (layer B.Cu) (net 17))
 (segment (start 130.82 107.32) (end 130.82 103.5) (width 0.254) (layer B.Cu) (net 17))
 (segment (start 129.96 113.5) (end 129.96 109) (width 0.254) (layer B.Cu) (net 13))
 (segment (start 129.96 109) (end 125.74 104.78) (width 0.254) (layer B.Cu) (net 13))
 (segment (start 125.74 104.78) (end 125.74 103.5) (width 0.254) (layer B.Cu) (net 13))
 (segment (start 127.42 113.5) (end 127.42 109) (width 0.254) (layer B.Cu) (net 9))
 (segment (start 127.42 109) (end 124.42 106) (width 0.254) (layer B.Cu) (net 9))
 (segment (start 124.42 106) (end 123.16 106) (width 0.254) (layer B.Cu) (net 9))
 (segment (start 123.16 106) (end 120.66 103.5) (width 0.254) (layer B.Cu) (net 9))
 (segment (start 124.88 113.5) (end 124.88 109) (width 0.254) (layer B.Cu) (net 5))
 (segment (start 124.88 109) (end 122.38 106.5) (width 0.254) (layer B.Cu) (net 5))
 (segment (start 122.38 106.5) (end 118.58 106.5) (width 0.254) (layer B.Cu) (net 5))
 (segment (start 118.58 106.5) (end 115.58 103.5) (width 0.254) (layer B.Cu) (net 5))
 (segment (start 104 98) (end 108.38 98) (width 0.254) (layer F.Cu) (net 18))
 (segment (start 108.38 98) (end 110.5 95.88) (width 0.254) (layer F.Cu) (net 18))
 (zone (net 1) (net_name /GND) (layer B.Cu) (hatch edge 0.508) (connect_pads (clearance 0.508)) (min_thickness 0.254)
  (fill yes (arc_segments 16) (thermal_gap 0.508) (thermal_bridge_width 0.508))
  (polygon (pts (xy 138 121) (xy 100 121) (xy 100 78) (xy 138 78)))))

